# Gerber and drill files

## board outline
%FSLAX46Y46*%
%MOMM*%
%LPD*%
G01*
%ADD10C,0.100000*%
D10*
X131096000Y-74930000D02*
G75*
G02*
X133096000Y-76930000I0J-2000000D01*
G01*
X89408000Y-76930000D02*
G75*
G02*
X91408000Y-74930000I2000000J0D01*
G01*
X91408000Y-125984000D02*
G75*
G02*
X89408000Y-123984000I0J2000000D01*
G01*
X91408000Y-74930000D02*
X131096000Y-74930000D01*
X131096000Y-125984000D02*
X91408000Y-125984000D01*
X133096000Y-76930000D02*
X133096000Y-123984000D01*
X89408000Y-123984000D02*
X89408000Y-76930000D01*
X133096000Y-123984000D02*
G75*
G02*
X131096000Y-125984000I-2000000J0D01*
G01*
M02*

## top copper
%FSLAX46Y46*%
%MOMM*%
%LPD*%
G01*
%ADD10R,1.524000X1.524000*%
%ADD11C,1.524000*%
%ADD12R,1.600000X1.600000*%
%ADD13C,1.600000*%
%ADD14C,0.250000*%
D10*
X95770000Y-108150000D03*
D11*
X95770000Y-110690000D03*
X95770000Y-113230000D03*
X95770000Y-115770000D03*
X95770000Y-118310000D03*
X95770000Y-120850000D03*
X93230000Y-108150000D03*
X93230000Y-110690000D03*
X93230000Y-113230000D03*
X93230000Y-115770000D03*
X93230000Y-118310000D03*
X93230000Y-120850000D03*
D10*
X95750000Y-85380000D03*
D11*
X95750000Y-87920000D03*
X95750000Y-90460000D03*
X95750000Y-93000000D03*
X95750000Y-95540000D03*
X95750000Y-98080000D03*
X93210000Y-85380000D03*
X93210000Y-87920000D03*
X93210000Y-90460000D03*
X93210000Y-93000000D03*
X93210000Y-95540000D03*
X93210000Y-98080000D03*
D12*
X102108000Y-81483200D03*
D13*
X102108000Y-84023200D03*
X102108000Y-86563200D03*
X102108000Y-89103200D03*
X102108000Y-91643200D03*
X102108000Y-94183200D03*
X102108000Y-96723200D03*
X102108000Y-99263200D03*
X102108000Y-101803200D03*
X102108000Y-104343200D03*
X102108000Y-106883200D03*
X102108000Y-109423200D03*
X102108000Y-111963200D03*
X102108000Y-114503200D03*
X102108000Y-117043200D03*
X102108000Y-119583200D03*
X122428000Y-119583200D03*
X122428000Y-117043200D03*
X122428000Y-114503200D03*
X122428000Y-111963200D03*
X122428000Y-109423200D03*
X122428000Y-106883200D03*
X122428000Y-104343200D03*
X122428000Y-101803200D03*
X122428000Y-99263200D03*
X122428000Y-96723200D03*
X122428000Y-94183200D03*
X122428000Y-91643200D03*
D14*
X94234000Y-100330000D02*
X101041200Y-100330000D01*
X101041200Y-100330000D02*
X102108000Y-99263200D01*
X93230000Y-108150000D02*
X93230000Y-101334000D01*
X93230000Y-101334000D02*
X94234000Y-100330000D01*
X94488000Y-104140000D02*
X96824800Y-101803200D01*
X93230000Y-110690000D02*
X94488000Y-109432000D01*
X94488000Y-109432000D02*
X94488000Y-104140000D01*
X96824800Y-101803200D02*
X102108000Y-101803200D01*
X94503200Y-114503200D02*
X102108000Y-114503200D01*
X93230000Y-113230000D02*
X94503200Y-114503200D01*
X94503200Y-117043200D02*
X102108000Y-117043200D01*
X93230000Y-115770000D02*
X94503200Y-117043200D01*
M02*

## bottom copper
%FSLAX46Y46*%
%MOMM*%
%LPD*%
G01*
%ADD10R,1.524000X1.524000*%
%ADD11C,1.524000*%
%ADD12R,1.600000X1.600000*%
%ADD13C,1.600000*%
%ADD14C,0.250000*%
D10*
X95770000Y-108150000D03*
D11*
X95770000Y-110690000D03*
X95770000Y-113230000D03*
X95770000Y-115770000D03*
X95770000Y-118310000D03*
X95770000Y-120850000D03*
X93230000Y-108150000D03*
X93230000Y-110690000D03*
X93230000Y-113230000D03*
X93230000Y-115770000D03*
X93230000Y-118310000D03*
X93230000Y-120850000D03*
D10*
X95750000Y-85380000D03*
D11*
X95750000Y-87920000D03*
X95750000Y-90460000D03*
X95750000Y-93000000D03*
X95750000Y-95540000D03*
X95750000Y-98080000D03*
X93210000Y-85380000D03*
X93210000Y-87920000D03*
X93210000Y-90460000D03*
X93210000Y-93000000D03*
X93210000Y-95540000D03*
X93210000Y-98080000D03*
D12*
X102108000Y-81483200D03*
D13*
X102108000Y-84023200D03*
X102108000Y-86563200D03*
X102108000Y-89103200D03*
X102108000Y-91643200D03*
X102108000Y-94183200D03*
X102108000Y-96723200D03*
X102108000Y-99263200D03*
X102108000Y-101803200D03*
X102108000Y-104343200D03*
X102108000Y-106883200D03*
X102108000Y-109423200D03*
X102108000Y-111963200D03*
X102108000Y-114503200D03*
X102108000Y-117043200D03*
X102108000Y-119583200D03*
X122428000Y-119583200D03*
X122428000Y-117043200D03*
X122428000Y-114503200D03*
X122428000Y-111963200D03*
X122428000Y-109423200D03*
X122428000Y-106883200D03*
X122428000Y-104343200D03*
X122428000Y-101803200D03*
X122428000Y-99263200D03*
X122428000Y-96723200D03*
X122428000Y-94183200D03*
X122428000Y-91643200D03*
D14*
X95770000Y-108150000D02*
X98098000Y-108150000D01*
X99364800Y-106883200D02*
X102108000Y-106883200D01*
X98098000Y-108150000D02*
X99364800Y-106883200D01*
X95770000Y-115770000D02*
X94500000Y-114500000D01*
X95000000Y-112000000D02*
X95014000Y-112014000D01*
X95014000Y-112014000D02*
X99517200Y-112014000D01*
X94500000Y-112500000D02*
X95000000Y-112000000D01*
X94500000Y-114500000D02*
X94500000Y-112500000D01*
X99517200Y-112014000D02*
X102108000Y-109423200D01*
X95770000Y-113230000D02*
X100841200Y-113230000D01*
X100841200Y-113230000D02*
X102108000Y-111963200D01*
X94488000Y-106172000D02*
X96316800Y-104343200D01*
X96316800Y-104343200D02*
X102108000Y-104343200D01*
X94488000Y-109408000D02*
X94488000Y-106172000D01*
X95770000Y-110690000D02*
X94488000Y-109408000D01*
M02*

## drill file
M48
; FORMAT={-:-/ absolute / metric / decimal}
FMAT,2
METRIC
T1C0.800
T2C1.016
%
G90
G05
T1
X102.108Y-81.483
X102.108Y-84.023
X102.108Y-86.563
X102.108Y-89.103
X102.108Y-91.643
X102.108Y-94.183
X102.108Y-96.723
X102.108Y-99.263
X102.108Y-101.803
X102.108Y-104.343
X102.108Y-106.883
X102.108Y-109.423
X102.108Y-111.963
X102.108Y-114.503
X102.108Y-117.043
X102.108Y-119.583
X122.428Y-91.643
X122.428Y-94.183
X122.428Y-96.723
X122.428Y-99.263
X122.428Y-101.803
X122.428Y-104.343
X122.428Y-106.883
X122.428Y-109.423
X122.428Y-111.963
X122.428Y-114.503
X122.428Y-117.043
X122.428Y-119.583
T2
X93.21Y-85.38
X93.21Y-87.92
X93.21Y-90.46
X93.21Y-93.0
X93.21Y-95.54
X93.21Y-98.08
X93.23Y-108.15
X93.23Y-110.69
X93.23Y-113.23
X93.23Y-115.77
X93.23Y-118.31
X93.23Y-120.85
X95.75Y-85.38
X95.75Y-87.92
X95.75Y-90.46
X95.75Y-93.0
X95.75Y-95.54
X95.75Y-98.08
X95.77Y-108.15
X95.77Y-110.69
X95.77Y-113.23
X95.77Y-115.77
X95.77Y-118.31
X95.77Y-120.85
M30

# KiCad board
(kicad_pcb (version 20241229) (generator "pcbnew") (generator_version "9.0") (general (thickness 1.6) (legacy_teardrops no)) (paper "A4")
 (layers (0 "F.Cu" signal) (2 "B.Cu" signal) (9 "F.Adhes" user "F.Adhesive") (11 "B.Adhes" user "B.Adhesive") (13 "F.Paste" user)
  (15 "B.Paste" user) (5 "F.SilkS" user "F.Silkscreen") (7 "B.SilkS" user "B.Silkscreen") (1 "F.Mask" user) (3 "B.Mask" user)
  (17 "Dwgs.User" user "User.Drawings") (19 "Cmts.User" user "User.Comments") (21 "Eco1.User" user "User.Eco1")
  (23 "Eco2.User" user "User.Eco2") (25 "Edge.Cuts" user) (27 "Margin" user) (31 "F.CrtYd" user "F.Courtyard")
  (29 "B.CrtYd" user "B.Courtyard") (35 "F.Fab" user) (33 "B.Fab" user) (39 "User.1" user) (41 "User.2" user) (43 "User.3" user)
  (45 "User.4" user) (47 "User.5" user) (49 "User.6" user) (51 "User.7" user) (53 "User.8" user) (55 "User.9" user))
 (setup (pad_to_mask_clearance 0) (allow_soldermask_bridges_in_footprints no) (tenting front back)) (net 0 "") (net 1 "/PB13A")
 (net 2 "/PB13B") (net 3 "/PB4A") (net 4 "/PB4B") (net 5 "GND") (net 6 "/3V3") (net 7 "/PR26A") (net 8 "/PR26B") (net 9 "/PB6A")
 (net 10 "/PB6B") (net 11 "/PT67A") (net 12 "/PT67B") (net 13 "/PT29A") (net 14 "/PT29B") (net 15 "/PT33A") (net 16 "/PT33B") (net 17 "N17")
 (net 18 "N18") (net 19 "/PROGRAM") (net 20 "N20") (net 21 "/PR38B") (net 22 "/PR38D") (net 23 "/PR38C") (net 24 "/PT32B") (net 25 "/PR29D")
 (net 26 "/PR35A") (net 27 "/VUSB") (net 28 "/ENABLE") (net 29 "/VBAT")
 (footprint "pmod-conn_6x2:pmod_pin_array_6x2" (layer "F.Cu") (at 94.5 114.5)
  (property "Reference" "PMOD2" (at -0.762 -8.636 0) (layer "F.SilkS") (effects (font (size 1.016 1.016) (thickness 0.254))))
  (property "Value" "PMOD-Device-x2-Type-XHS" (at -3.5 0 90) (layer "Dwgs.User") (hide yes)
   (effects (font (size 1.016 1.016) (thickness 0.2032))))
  (pad "1" thru_hole rect (at 1.27 -6.35) (size 1.524 1.524) (drill 1.016) (layers "*.Cu" "*.Mask" "F.SilkS") (remove_unused_layers no)
   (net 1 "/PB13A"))
  (pad "2" thru_hole circle (at 1.27 -3.81 270) (size 1.524 1.524) (drill 1.016) (layers "*.Cu" "*.Mask" "F.SilkS")
   (remove_unused_layers no) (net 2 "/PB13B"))
  (pad "3" thru_hole circle (at 1.27 -1.27 270) (size 1.524 1.524) (drill 1.016) (layers "*.Cu" "*.Mask" "F.SilkS")
   (remove_unused_layers no) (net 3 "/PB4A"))
  (pad "4" thru_hole circle (at 1.27 1.27 270) (size 1.524 1.524) (drill 1.016) (layers "*.Cu" "*.Mask" "F.SilkS") (remove_unused_layers no)
   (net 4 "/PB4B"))
  (pad "5" thru_hole circle (at 1.27 3.81 270) (size 1.524 1.524) (drill 1.016) (layers "*.Cu" "*.Mask" "F.SilkS") (remove_unused_layers no)
   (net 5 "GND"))
  (pad "6" thru_hole circle (at 1.27 6.35 270) (size 1.524 1.524) (drill 1.016) (layers "*.Cu" "*.Mask" "F.SilkS") (remove_unused_layers no)
   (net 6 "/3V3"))
  (pad "7" thru_hole circle (at -1.27 -6.35 270) (size 1.524 1.524) (drill 1.016) (layers "*.Cu" "*.Mask" "F.SilkS")
   (remove_unused_layers no) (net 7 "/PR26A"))
  (pad "8" thru_hole circle (at -1.27 -3.81 270) (size 1.524 1.524) (drill 1.016) (layers "*.Cu" "*.Mask" "F.SilkS")
   (remove_unused_layers no) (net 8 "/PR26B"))
  (pad "9" thru_hole circle (at -1.27 -1.27 270) (size 1.524 1.524) (drill 1.016) (layers "*.Cu" "*.Mask" "F.SilkS")
   (remove_unused_layers no) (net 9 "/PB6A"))
  (pad "10" thru_hole circle (at -1.27 1.27 270) (size 1.524 1.524) (drill 1.016) (layers "*.Cu" "*.Mask" "F.SilkS")
   (remove_unused_layers no) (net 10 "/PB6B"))
  (pad "11" thru_hole circle (at -1.27 3.81 270) (size 1.524 1.524) (drill 1.016) (layers "*.Cu" "*.Mask" "F.SilkS")
   (remove_unused_layers no) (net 5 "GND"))
  (pad "12" thru_hole circle (at -1.27 6.35 270) (size 1.524 1.524) (drill 1.016) (layers "*.Cu" "*.Mask" "F.SilkS")
   (remove_unused_layers no) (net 6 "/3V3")))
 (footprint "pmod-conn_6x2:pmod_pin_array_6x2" (layer "F.Cu") (at 94.48 91.73)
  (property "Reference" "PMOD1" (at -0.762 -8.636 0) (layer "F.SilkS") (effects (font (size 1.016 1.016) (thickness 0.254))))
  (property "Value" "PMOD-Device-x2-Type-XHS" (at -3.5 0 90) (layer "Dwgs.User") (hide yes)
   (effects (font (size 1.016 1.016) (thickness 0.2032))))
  (pad "1" thru_hole rect (at 1.27 -6.35) (size 1.524 1.524) (drill 1.016) (layers "*.Cu" "*.Mask" "F.SilkS") (remove_unused_layers no)
   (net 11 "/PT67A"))
  (pad "2" thru_hole circle (at 1.27 -3.81 270) (size 1.524 1.524) (drill 1.016) (layers "*.Cu" "*.Mask" "F.SilkS")
   (remove_unused_layers no) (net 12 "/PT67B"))
  (pad "3" thru_hole circle (at 1.27 -1.27 270) (size 1.524 1.524) (drill 1.016) (layers "*.Cu" "*.Mask" "F.SilkS")
   (remove_unused_layers no) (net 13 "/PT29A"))
  (pad "4" thru_hole circle (at 1.27 1.27 270) (size 1.524 1.524) (drill 1.016) (layers "*.Cu" "*.Mask" "F.SilkS") (remove_unused_layers no)
   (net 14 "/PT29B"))
  (pad "5" thru_hole circle (at 1.27 3.81 270) (size 1.524 1.524) (drill 1.016) (layers "*.Cu" "*.Mask" "F.SilkS") (remove_unused_layers no)
   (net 5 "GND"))
  (pad "6" thru_hole circle (at 1.27 6.35 270) (size 1.524 1.524) (drill 1.016) (layers "*.Cu" "*.Mask" "F.SilkS") (remove_unused_layers no)
   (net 6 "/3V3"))
  (pad "7" thru_hole circle (at -1.27 -6.35 270) (size 1.524 1.524) (drill 1.016) (layers "*.Cu" "*.Mask" "F.SilkS")
   (remove_unused_layers no) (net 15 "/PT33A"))
  (pad "8" thru_hole circle (at -1.27 -3.81 270) (size 1.524 1.524) (drill 1.016) (layers "*.Cu" "*.Mask" "F.SilkS")
   (remove_unused_layers no) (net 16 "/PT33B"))
  (pad "9" thru_hole circle (at -1.27 -1.27 270) (size 1.524 1.524) (drill 1.016) (layers "*.Cu" "*.Mask" "F.SilkS")
   (remove_unused_layers no) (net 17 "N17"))
  (pad "10" thru_hole circle (at -1.27 1.27 270) (size 1.524 1.524) (drill 1.016) (layers "*.Cu" "*.Mask" "F.SilkS")
   (remove_unused_layers no) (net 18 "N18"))
  (pad "11" thru_hole circle (at -1.27 3.81 270) (size 1.524 1.524) (drill 1.016) (layers "*.Cu" "*.Mask" "F.SilkS")
   (remove_unused_layers no) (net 5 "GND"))
  (pad "12" thru_hole circle (at -1.27 6.35 270) (size 1.524 1.524) (drill 1.016) (layers "*.Cu" "*.Mask" "F.SilkS")
   (remove_unused_layers no) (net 6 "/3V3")))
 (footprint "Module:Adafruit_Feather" (layer "F.Cu") (at 102.108 81.4832)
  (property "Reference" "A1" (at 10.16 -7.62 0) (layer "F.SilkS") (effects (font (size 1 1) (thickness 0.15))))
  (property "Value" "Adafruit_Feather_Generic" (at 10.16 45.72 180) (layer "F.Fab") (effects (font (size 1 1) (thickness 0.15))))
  (pad "1" thru_hole rect (at 0 0 180) (size 1.6 1.6) (drill 0.8) (layers "*.Cu" "*.Mask") (remove_unused_layers no) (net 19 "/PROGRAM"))
  (pad "2" thru_hole circle (at 0 2.54 180) (size 1.6 1.6) (drill 0.8) (layers "*.Cu" "*.Mask") (remove_unused_layers no) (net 6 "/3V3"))
  (pad "3" thru_hole circle (at 0 5.08 180) (size 1.6 1.6) (drill 0.8) (layers "*.Cu" "*.Mask") (remove_unused_layers no) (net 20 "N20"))
  (pad "4" thru_hole circle (at 0 7.62 180) (size 1.6 1.6) (drill 0.8) (layers "*.Cu" "*.Mask") (remove_unused_layers no) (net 5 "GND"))
  (pad "5" thru_hole circle (at 0 10.16 180) (size 1.6 1.6) (drill 0.8) (layers "*.Cu" "*.Mask") (remove_unused_layers no) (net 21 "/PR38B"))
  (pad "6" thru_hole circle (at 0 12.7 180) (size 1.6 1.6) (drill 0.8) (layers "*.Cu" "*.Mask") (remove_unused_layers no) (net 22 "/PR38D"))
  (pad "7" thru_hole circle (at 0 15.24 180) (size 1.6 1.6) (drill 0.8) (layers "*.Cu" "*.Mask") (remove_unused_layers no) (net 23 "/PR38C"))
  (pad "8" thru_hole circle (at 0 17.78 180) (size 1.6 1.6) (drill 0.8) (layers "*.Cu" "*.Mask") (remove_unused_layers no) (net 7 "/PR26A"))
  (pad "9" thru_hole circle (at 0 20.32 180) (size 1.6 1.6) (drill 0.8) (layers "*.Cu" "*.Mask") (remove_unused_layers no) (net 8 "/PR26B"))
  (pad "10" thru_hole circle (at 0 22.86 180) (size 1.6 1.6) (drill 0.8) (layers "*.Cu" "*.Mask") (remove_unused_layers no) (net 2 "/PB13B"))
  (pad "11" thru_hole circle (at 0 25.4 180) (size 1.6 1.6) (drill 0.8) (layers "*.Cu" "*.Mask") (remove_unused_layers no) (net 1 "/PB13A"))
  (pad "12" thru_hole circle (at 0 27.94 180) (size 1.6 1.6) (drill 0.8) (layers "*.Cu" "*.Mask") (remove_unused_layers no) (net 4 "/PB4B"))
  (pad "13" thru_hole circle (at 0 30.48 180) (size 1.6 1.6) (drill 0.8) (layers "*.Cu" "*.Mask") (remove_unused_layers no) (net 3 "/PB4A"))
  (pad "14" thru_hole circle (at 0 33.02 180) (size 1.6 1.6) (drill 0.8) (layers "*.Cu" "*.Mask") (remove_unused_layers no) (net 9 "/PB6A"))
  (pad "15" thru_hole circle (at 0 35.56 180) (size 1.6 1.6) (drill 0.8) (layers "*.Cu" "*.Mask") (remove_unused_layers no) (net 10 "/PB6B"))
  (pad "16" thru_hole circle (at 0 38.1 180) (size 1.6 1.6) (drill 0.8) (layers "*.Cu" "*.Mask") (remove_unused_layers no) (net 5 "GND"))
  (pad "17" thru_hole circle (at 20.32 38.1 180) (size 1.6 1.6) (drill 0.8) (layers "*.Cu" "*.Mask") (remove_unused_layers no)
   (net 14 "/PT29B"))
  (pad "18" thru_hole circle (at 20.32 35.56 180) (size 1.6 1.6) (drill 0.8) (layers "*.Cu" "*.Mask") (remove_unused_layers no)
   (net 16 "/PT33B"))
  (pad "19" thru_hole circle (at 20.32 33.02 180) (size 1.6 1.6) (drill 0.8) (layers "*.Cu" "*.Mask") (remove_unused_layers no)
   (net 13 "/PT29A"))
  (pad "20" thru_hole circle (at 20.32 30.48 180) (size 1.6 1.6) (drill 0.8) (layers "*.Cu" "*.Mask") (remove_unused_layers no)
   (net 15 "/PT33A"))
  (pad "21" thru_hole circle (at 20.32 27.94 180) (size 1.6 1.6) (drill 0.8) (layers "*.Cu" "*.Mask") (remove_unused_layers no)
   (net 12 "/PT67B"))
  (pad "22" thru_hole circle (at 20.32 25.4 180) (size 1.6 1.6) (drill 0.8) (layers "*.Cu" "*.Mask") (remove_unused_layers no)
   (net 11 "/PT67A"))
  (pad "23" thru_hole circle (at 20.32 22.86 180) (size 1.6 1.6) (drill 0.8) (layers "*.Cu" "*.Mask") (remove_unused_layers no)
   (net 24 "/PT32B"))
  (pad "24" thru_hole circle (at 20.32 20.32 180) (size 1.6 1.6) (drill 0.8) (layers "*.Cu" "*.Mask") (remove_unused_layers no)
   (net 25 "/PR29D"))
  (pad "25" thru_hole circle (at 20.32 17.78 180) (size 1.6 1.6) (drill 0.8) (layers "*.Cu" "*.Mask") (remove_unused_layers no)
   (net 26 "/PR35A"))
  (pad "26" thru_hole circle (at 20.32 15.24 180) (size 1.6 1.6) (drill 0.8) (layers "*.Cu" "*.Mask") (remove_unused_layers no)
   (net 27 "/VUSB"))
  (pad "27" thru_hole circle (at 20.32 12.7 180) (size 1.6 1.6) (drill 0.8) (layers "*.Cu" "*.Mask") (remove_unused_layers no)
   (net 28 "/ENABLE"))
  (pad "28" thru_hole circle (at 20.32 10.16 180) (size 1.6 1.6) (drill 0.8) (layers "*.Cu" "*.Mask") (remove_unused_layers no)
   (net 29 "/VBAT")))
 (gr_arc (start 131.096 74.93) (mid 132.510214 75.515786) (end 133.096 76.93) (stroke (width 0.1) (type default)) (layer "Edge.Cuts"))
 (gr_arc (start 89.408 76.93) (mid 89.993786 75.515786) (end 91.408 74.93) (stroke (width 0.1) (type default)) (layer "Edge.Cuts"))
 (gr_arc (start 91.408 125.984) (mid 89.993786 125.398214) (end 89.408 123.984) (stroke (width 0.1) (type default)) (layer "Edge.Cuts"))
 (gr_line (start 91.408 74.93) (end 131.096 74.93) (stroke (width 0.1) (type default)) (layer "Edge.Cuts"))
 (gr_line (start 131.096 125.984) (end 91.408 125.984) (stroke (width 0.1) (type default)) (layer "Edge.Cuts"))
 (gr_line (start 133.096 76.93) (end 133.096 123.984) (stroke (width 0.1) (type default)) (layer "Edge.Cuts"))
 (gr_line (start 89.408 123.984) (end 89.408 76.93) (stroke (width 0.1) (type default)) (layer "Edge.Cuts"))
 (gr_arc (start 133.096 123.984) (mid 132.510214 125.398214) (end 131.096 125.984) (stroke (width 0.1) (type default)) (layer "Edge.Cuts"))
 (segment (start 94.234 100.33) (end 101.0412 100.33) (width 0.25) (layer "F.Cu") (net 7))
 (segment (start 101.0412 100.33) (end 102.108 99.2632) (width 0.25) (layer "F.Cu") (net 7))
 (segment (start 93.23 108.15) (end 93.23 101.334) (width 0.25) (layer "F.Cu") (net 7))
 (segment (start 93.23 101.334) (end 94.234 100.33) (width 0.25) (layer "F.Cu") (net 7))
 (segment (start 94.488 104.14) (end 96.8248 101.8032) (width 0.25) (layer "F.Cu") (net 8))
 (segment (start 93.23 110.69) (end 94.488 109.432) (width 0.25) (layer "F.Cu") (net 8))
 (segment (start 94.488 109.432) (end 94.488 104.14) (width 0.25) (layer "F.Cu") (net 8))
 (segment (start 96.8248 101.8032) (end 102.108 101.8032) (width 0.25) (layer "F.Cu") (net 8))
 (segment (start 95.77 108.15) (end 98.098 108.15) (width 0.25) (layer "B.Cu") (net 1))
 (segment (start 99.3648 106.8832) (end 102.108 106.8832) (width 0.25) (layer "B.Cu") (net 1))
 (segment (start 98.098 108.15) (end 99.3648 106.8832) (width 0.25) (layer "B.Cu") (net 1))
 (segment (start 95.77 115.77) (end 94.5 114.5) (width 0.25) (layer "B.Cu") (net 4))
 (segment (start 95 112) (end 95.014 112.014) (width 0.25) (layer "B.Cu") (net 4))
 (segment (start 95.014 112.014) (end 99.5172 112.014) (width 0.25) (layer "B.Cu") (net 4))
 (segment (start 94.5 112.5) (end 95 112) (width 0.25) (layer "B.Cu") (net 4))
 (segment (start 94.5 114.5) (end 94.5 112.5) (width 0.25) (layer "B.Cu") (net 4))
 (segment (start 99.5172 112.014) (end 102.108 109.4232) (width 0.25) (layer "B.Cu") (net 4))
 (segment (start 95.77 113.23) (end 100.8412 113.23) (width 0.25) (layer "B.Cu") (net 3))
 (segment (start 100.8412 113.23) (end 102.108 111.9632) (width 0.25) (layer "B.Cu") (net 3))
 (segment (start 94.488 106.172) (end 96.3168 104.3432) (width 0.25) (layer "B.Cu") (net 2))
 (segment (start 96.3168 104.3432) (end 102.108 104.3432) (width 0.25) (layer "B.Cu") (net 2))
 (segment (start 94.488 109.408) (end 94.488 106.172) (width 0.25) (layer "B.Cu") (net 2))
 (segment (start 95.77 110.69) (end 94.488 109.408) (width 0.25) (layer "B.Cu") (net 2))
 (segment (start 94.5032 114.5032) (end 102.108 114.5032) (width 0.25) (layer "F.Cu") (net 9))
 (segment (start 93.23 113.23) (end 94.5032 114.5032) (width 0.25) (layer "F.Cu") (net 9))
 (segment (start 94.5032 117.0432) (end 102.108 117.0432) (width 0.25) (layer "F.Cu") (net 10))
 (segment (start 93.23 115.77) (end 94.5032 117.0432) (width 0.25) (layer "F.Cu") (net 10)))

